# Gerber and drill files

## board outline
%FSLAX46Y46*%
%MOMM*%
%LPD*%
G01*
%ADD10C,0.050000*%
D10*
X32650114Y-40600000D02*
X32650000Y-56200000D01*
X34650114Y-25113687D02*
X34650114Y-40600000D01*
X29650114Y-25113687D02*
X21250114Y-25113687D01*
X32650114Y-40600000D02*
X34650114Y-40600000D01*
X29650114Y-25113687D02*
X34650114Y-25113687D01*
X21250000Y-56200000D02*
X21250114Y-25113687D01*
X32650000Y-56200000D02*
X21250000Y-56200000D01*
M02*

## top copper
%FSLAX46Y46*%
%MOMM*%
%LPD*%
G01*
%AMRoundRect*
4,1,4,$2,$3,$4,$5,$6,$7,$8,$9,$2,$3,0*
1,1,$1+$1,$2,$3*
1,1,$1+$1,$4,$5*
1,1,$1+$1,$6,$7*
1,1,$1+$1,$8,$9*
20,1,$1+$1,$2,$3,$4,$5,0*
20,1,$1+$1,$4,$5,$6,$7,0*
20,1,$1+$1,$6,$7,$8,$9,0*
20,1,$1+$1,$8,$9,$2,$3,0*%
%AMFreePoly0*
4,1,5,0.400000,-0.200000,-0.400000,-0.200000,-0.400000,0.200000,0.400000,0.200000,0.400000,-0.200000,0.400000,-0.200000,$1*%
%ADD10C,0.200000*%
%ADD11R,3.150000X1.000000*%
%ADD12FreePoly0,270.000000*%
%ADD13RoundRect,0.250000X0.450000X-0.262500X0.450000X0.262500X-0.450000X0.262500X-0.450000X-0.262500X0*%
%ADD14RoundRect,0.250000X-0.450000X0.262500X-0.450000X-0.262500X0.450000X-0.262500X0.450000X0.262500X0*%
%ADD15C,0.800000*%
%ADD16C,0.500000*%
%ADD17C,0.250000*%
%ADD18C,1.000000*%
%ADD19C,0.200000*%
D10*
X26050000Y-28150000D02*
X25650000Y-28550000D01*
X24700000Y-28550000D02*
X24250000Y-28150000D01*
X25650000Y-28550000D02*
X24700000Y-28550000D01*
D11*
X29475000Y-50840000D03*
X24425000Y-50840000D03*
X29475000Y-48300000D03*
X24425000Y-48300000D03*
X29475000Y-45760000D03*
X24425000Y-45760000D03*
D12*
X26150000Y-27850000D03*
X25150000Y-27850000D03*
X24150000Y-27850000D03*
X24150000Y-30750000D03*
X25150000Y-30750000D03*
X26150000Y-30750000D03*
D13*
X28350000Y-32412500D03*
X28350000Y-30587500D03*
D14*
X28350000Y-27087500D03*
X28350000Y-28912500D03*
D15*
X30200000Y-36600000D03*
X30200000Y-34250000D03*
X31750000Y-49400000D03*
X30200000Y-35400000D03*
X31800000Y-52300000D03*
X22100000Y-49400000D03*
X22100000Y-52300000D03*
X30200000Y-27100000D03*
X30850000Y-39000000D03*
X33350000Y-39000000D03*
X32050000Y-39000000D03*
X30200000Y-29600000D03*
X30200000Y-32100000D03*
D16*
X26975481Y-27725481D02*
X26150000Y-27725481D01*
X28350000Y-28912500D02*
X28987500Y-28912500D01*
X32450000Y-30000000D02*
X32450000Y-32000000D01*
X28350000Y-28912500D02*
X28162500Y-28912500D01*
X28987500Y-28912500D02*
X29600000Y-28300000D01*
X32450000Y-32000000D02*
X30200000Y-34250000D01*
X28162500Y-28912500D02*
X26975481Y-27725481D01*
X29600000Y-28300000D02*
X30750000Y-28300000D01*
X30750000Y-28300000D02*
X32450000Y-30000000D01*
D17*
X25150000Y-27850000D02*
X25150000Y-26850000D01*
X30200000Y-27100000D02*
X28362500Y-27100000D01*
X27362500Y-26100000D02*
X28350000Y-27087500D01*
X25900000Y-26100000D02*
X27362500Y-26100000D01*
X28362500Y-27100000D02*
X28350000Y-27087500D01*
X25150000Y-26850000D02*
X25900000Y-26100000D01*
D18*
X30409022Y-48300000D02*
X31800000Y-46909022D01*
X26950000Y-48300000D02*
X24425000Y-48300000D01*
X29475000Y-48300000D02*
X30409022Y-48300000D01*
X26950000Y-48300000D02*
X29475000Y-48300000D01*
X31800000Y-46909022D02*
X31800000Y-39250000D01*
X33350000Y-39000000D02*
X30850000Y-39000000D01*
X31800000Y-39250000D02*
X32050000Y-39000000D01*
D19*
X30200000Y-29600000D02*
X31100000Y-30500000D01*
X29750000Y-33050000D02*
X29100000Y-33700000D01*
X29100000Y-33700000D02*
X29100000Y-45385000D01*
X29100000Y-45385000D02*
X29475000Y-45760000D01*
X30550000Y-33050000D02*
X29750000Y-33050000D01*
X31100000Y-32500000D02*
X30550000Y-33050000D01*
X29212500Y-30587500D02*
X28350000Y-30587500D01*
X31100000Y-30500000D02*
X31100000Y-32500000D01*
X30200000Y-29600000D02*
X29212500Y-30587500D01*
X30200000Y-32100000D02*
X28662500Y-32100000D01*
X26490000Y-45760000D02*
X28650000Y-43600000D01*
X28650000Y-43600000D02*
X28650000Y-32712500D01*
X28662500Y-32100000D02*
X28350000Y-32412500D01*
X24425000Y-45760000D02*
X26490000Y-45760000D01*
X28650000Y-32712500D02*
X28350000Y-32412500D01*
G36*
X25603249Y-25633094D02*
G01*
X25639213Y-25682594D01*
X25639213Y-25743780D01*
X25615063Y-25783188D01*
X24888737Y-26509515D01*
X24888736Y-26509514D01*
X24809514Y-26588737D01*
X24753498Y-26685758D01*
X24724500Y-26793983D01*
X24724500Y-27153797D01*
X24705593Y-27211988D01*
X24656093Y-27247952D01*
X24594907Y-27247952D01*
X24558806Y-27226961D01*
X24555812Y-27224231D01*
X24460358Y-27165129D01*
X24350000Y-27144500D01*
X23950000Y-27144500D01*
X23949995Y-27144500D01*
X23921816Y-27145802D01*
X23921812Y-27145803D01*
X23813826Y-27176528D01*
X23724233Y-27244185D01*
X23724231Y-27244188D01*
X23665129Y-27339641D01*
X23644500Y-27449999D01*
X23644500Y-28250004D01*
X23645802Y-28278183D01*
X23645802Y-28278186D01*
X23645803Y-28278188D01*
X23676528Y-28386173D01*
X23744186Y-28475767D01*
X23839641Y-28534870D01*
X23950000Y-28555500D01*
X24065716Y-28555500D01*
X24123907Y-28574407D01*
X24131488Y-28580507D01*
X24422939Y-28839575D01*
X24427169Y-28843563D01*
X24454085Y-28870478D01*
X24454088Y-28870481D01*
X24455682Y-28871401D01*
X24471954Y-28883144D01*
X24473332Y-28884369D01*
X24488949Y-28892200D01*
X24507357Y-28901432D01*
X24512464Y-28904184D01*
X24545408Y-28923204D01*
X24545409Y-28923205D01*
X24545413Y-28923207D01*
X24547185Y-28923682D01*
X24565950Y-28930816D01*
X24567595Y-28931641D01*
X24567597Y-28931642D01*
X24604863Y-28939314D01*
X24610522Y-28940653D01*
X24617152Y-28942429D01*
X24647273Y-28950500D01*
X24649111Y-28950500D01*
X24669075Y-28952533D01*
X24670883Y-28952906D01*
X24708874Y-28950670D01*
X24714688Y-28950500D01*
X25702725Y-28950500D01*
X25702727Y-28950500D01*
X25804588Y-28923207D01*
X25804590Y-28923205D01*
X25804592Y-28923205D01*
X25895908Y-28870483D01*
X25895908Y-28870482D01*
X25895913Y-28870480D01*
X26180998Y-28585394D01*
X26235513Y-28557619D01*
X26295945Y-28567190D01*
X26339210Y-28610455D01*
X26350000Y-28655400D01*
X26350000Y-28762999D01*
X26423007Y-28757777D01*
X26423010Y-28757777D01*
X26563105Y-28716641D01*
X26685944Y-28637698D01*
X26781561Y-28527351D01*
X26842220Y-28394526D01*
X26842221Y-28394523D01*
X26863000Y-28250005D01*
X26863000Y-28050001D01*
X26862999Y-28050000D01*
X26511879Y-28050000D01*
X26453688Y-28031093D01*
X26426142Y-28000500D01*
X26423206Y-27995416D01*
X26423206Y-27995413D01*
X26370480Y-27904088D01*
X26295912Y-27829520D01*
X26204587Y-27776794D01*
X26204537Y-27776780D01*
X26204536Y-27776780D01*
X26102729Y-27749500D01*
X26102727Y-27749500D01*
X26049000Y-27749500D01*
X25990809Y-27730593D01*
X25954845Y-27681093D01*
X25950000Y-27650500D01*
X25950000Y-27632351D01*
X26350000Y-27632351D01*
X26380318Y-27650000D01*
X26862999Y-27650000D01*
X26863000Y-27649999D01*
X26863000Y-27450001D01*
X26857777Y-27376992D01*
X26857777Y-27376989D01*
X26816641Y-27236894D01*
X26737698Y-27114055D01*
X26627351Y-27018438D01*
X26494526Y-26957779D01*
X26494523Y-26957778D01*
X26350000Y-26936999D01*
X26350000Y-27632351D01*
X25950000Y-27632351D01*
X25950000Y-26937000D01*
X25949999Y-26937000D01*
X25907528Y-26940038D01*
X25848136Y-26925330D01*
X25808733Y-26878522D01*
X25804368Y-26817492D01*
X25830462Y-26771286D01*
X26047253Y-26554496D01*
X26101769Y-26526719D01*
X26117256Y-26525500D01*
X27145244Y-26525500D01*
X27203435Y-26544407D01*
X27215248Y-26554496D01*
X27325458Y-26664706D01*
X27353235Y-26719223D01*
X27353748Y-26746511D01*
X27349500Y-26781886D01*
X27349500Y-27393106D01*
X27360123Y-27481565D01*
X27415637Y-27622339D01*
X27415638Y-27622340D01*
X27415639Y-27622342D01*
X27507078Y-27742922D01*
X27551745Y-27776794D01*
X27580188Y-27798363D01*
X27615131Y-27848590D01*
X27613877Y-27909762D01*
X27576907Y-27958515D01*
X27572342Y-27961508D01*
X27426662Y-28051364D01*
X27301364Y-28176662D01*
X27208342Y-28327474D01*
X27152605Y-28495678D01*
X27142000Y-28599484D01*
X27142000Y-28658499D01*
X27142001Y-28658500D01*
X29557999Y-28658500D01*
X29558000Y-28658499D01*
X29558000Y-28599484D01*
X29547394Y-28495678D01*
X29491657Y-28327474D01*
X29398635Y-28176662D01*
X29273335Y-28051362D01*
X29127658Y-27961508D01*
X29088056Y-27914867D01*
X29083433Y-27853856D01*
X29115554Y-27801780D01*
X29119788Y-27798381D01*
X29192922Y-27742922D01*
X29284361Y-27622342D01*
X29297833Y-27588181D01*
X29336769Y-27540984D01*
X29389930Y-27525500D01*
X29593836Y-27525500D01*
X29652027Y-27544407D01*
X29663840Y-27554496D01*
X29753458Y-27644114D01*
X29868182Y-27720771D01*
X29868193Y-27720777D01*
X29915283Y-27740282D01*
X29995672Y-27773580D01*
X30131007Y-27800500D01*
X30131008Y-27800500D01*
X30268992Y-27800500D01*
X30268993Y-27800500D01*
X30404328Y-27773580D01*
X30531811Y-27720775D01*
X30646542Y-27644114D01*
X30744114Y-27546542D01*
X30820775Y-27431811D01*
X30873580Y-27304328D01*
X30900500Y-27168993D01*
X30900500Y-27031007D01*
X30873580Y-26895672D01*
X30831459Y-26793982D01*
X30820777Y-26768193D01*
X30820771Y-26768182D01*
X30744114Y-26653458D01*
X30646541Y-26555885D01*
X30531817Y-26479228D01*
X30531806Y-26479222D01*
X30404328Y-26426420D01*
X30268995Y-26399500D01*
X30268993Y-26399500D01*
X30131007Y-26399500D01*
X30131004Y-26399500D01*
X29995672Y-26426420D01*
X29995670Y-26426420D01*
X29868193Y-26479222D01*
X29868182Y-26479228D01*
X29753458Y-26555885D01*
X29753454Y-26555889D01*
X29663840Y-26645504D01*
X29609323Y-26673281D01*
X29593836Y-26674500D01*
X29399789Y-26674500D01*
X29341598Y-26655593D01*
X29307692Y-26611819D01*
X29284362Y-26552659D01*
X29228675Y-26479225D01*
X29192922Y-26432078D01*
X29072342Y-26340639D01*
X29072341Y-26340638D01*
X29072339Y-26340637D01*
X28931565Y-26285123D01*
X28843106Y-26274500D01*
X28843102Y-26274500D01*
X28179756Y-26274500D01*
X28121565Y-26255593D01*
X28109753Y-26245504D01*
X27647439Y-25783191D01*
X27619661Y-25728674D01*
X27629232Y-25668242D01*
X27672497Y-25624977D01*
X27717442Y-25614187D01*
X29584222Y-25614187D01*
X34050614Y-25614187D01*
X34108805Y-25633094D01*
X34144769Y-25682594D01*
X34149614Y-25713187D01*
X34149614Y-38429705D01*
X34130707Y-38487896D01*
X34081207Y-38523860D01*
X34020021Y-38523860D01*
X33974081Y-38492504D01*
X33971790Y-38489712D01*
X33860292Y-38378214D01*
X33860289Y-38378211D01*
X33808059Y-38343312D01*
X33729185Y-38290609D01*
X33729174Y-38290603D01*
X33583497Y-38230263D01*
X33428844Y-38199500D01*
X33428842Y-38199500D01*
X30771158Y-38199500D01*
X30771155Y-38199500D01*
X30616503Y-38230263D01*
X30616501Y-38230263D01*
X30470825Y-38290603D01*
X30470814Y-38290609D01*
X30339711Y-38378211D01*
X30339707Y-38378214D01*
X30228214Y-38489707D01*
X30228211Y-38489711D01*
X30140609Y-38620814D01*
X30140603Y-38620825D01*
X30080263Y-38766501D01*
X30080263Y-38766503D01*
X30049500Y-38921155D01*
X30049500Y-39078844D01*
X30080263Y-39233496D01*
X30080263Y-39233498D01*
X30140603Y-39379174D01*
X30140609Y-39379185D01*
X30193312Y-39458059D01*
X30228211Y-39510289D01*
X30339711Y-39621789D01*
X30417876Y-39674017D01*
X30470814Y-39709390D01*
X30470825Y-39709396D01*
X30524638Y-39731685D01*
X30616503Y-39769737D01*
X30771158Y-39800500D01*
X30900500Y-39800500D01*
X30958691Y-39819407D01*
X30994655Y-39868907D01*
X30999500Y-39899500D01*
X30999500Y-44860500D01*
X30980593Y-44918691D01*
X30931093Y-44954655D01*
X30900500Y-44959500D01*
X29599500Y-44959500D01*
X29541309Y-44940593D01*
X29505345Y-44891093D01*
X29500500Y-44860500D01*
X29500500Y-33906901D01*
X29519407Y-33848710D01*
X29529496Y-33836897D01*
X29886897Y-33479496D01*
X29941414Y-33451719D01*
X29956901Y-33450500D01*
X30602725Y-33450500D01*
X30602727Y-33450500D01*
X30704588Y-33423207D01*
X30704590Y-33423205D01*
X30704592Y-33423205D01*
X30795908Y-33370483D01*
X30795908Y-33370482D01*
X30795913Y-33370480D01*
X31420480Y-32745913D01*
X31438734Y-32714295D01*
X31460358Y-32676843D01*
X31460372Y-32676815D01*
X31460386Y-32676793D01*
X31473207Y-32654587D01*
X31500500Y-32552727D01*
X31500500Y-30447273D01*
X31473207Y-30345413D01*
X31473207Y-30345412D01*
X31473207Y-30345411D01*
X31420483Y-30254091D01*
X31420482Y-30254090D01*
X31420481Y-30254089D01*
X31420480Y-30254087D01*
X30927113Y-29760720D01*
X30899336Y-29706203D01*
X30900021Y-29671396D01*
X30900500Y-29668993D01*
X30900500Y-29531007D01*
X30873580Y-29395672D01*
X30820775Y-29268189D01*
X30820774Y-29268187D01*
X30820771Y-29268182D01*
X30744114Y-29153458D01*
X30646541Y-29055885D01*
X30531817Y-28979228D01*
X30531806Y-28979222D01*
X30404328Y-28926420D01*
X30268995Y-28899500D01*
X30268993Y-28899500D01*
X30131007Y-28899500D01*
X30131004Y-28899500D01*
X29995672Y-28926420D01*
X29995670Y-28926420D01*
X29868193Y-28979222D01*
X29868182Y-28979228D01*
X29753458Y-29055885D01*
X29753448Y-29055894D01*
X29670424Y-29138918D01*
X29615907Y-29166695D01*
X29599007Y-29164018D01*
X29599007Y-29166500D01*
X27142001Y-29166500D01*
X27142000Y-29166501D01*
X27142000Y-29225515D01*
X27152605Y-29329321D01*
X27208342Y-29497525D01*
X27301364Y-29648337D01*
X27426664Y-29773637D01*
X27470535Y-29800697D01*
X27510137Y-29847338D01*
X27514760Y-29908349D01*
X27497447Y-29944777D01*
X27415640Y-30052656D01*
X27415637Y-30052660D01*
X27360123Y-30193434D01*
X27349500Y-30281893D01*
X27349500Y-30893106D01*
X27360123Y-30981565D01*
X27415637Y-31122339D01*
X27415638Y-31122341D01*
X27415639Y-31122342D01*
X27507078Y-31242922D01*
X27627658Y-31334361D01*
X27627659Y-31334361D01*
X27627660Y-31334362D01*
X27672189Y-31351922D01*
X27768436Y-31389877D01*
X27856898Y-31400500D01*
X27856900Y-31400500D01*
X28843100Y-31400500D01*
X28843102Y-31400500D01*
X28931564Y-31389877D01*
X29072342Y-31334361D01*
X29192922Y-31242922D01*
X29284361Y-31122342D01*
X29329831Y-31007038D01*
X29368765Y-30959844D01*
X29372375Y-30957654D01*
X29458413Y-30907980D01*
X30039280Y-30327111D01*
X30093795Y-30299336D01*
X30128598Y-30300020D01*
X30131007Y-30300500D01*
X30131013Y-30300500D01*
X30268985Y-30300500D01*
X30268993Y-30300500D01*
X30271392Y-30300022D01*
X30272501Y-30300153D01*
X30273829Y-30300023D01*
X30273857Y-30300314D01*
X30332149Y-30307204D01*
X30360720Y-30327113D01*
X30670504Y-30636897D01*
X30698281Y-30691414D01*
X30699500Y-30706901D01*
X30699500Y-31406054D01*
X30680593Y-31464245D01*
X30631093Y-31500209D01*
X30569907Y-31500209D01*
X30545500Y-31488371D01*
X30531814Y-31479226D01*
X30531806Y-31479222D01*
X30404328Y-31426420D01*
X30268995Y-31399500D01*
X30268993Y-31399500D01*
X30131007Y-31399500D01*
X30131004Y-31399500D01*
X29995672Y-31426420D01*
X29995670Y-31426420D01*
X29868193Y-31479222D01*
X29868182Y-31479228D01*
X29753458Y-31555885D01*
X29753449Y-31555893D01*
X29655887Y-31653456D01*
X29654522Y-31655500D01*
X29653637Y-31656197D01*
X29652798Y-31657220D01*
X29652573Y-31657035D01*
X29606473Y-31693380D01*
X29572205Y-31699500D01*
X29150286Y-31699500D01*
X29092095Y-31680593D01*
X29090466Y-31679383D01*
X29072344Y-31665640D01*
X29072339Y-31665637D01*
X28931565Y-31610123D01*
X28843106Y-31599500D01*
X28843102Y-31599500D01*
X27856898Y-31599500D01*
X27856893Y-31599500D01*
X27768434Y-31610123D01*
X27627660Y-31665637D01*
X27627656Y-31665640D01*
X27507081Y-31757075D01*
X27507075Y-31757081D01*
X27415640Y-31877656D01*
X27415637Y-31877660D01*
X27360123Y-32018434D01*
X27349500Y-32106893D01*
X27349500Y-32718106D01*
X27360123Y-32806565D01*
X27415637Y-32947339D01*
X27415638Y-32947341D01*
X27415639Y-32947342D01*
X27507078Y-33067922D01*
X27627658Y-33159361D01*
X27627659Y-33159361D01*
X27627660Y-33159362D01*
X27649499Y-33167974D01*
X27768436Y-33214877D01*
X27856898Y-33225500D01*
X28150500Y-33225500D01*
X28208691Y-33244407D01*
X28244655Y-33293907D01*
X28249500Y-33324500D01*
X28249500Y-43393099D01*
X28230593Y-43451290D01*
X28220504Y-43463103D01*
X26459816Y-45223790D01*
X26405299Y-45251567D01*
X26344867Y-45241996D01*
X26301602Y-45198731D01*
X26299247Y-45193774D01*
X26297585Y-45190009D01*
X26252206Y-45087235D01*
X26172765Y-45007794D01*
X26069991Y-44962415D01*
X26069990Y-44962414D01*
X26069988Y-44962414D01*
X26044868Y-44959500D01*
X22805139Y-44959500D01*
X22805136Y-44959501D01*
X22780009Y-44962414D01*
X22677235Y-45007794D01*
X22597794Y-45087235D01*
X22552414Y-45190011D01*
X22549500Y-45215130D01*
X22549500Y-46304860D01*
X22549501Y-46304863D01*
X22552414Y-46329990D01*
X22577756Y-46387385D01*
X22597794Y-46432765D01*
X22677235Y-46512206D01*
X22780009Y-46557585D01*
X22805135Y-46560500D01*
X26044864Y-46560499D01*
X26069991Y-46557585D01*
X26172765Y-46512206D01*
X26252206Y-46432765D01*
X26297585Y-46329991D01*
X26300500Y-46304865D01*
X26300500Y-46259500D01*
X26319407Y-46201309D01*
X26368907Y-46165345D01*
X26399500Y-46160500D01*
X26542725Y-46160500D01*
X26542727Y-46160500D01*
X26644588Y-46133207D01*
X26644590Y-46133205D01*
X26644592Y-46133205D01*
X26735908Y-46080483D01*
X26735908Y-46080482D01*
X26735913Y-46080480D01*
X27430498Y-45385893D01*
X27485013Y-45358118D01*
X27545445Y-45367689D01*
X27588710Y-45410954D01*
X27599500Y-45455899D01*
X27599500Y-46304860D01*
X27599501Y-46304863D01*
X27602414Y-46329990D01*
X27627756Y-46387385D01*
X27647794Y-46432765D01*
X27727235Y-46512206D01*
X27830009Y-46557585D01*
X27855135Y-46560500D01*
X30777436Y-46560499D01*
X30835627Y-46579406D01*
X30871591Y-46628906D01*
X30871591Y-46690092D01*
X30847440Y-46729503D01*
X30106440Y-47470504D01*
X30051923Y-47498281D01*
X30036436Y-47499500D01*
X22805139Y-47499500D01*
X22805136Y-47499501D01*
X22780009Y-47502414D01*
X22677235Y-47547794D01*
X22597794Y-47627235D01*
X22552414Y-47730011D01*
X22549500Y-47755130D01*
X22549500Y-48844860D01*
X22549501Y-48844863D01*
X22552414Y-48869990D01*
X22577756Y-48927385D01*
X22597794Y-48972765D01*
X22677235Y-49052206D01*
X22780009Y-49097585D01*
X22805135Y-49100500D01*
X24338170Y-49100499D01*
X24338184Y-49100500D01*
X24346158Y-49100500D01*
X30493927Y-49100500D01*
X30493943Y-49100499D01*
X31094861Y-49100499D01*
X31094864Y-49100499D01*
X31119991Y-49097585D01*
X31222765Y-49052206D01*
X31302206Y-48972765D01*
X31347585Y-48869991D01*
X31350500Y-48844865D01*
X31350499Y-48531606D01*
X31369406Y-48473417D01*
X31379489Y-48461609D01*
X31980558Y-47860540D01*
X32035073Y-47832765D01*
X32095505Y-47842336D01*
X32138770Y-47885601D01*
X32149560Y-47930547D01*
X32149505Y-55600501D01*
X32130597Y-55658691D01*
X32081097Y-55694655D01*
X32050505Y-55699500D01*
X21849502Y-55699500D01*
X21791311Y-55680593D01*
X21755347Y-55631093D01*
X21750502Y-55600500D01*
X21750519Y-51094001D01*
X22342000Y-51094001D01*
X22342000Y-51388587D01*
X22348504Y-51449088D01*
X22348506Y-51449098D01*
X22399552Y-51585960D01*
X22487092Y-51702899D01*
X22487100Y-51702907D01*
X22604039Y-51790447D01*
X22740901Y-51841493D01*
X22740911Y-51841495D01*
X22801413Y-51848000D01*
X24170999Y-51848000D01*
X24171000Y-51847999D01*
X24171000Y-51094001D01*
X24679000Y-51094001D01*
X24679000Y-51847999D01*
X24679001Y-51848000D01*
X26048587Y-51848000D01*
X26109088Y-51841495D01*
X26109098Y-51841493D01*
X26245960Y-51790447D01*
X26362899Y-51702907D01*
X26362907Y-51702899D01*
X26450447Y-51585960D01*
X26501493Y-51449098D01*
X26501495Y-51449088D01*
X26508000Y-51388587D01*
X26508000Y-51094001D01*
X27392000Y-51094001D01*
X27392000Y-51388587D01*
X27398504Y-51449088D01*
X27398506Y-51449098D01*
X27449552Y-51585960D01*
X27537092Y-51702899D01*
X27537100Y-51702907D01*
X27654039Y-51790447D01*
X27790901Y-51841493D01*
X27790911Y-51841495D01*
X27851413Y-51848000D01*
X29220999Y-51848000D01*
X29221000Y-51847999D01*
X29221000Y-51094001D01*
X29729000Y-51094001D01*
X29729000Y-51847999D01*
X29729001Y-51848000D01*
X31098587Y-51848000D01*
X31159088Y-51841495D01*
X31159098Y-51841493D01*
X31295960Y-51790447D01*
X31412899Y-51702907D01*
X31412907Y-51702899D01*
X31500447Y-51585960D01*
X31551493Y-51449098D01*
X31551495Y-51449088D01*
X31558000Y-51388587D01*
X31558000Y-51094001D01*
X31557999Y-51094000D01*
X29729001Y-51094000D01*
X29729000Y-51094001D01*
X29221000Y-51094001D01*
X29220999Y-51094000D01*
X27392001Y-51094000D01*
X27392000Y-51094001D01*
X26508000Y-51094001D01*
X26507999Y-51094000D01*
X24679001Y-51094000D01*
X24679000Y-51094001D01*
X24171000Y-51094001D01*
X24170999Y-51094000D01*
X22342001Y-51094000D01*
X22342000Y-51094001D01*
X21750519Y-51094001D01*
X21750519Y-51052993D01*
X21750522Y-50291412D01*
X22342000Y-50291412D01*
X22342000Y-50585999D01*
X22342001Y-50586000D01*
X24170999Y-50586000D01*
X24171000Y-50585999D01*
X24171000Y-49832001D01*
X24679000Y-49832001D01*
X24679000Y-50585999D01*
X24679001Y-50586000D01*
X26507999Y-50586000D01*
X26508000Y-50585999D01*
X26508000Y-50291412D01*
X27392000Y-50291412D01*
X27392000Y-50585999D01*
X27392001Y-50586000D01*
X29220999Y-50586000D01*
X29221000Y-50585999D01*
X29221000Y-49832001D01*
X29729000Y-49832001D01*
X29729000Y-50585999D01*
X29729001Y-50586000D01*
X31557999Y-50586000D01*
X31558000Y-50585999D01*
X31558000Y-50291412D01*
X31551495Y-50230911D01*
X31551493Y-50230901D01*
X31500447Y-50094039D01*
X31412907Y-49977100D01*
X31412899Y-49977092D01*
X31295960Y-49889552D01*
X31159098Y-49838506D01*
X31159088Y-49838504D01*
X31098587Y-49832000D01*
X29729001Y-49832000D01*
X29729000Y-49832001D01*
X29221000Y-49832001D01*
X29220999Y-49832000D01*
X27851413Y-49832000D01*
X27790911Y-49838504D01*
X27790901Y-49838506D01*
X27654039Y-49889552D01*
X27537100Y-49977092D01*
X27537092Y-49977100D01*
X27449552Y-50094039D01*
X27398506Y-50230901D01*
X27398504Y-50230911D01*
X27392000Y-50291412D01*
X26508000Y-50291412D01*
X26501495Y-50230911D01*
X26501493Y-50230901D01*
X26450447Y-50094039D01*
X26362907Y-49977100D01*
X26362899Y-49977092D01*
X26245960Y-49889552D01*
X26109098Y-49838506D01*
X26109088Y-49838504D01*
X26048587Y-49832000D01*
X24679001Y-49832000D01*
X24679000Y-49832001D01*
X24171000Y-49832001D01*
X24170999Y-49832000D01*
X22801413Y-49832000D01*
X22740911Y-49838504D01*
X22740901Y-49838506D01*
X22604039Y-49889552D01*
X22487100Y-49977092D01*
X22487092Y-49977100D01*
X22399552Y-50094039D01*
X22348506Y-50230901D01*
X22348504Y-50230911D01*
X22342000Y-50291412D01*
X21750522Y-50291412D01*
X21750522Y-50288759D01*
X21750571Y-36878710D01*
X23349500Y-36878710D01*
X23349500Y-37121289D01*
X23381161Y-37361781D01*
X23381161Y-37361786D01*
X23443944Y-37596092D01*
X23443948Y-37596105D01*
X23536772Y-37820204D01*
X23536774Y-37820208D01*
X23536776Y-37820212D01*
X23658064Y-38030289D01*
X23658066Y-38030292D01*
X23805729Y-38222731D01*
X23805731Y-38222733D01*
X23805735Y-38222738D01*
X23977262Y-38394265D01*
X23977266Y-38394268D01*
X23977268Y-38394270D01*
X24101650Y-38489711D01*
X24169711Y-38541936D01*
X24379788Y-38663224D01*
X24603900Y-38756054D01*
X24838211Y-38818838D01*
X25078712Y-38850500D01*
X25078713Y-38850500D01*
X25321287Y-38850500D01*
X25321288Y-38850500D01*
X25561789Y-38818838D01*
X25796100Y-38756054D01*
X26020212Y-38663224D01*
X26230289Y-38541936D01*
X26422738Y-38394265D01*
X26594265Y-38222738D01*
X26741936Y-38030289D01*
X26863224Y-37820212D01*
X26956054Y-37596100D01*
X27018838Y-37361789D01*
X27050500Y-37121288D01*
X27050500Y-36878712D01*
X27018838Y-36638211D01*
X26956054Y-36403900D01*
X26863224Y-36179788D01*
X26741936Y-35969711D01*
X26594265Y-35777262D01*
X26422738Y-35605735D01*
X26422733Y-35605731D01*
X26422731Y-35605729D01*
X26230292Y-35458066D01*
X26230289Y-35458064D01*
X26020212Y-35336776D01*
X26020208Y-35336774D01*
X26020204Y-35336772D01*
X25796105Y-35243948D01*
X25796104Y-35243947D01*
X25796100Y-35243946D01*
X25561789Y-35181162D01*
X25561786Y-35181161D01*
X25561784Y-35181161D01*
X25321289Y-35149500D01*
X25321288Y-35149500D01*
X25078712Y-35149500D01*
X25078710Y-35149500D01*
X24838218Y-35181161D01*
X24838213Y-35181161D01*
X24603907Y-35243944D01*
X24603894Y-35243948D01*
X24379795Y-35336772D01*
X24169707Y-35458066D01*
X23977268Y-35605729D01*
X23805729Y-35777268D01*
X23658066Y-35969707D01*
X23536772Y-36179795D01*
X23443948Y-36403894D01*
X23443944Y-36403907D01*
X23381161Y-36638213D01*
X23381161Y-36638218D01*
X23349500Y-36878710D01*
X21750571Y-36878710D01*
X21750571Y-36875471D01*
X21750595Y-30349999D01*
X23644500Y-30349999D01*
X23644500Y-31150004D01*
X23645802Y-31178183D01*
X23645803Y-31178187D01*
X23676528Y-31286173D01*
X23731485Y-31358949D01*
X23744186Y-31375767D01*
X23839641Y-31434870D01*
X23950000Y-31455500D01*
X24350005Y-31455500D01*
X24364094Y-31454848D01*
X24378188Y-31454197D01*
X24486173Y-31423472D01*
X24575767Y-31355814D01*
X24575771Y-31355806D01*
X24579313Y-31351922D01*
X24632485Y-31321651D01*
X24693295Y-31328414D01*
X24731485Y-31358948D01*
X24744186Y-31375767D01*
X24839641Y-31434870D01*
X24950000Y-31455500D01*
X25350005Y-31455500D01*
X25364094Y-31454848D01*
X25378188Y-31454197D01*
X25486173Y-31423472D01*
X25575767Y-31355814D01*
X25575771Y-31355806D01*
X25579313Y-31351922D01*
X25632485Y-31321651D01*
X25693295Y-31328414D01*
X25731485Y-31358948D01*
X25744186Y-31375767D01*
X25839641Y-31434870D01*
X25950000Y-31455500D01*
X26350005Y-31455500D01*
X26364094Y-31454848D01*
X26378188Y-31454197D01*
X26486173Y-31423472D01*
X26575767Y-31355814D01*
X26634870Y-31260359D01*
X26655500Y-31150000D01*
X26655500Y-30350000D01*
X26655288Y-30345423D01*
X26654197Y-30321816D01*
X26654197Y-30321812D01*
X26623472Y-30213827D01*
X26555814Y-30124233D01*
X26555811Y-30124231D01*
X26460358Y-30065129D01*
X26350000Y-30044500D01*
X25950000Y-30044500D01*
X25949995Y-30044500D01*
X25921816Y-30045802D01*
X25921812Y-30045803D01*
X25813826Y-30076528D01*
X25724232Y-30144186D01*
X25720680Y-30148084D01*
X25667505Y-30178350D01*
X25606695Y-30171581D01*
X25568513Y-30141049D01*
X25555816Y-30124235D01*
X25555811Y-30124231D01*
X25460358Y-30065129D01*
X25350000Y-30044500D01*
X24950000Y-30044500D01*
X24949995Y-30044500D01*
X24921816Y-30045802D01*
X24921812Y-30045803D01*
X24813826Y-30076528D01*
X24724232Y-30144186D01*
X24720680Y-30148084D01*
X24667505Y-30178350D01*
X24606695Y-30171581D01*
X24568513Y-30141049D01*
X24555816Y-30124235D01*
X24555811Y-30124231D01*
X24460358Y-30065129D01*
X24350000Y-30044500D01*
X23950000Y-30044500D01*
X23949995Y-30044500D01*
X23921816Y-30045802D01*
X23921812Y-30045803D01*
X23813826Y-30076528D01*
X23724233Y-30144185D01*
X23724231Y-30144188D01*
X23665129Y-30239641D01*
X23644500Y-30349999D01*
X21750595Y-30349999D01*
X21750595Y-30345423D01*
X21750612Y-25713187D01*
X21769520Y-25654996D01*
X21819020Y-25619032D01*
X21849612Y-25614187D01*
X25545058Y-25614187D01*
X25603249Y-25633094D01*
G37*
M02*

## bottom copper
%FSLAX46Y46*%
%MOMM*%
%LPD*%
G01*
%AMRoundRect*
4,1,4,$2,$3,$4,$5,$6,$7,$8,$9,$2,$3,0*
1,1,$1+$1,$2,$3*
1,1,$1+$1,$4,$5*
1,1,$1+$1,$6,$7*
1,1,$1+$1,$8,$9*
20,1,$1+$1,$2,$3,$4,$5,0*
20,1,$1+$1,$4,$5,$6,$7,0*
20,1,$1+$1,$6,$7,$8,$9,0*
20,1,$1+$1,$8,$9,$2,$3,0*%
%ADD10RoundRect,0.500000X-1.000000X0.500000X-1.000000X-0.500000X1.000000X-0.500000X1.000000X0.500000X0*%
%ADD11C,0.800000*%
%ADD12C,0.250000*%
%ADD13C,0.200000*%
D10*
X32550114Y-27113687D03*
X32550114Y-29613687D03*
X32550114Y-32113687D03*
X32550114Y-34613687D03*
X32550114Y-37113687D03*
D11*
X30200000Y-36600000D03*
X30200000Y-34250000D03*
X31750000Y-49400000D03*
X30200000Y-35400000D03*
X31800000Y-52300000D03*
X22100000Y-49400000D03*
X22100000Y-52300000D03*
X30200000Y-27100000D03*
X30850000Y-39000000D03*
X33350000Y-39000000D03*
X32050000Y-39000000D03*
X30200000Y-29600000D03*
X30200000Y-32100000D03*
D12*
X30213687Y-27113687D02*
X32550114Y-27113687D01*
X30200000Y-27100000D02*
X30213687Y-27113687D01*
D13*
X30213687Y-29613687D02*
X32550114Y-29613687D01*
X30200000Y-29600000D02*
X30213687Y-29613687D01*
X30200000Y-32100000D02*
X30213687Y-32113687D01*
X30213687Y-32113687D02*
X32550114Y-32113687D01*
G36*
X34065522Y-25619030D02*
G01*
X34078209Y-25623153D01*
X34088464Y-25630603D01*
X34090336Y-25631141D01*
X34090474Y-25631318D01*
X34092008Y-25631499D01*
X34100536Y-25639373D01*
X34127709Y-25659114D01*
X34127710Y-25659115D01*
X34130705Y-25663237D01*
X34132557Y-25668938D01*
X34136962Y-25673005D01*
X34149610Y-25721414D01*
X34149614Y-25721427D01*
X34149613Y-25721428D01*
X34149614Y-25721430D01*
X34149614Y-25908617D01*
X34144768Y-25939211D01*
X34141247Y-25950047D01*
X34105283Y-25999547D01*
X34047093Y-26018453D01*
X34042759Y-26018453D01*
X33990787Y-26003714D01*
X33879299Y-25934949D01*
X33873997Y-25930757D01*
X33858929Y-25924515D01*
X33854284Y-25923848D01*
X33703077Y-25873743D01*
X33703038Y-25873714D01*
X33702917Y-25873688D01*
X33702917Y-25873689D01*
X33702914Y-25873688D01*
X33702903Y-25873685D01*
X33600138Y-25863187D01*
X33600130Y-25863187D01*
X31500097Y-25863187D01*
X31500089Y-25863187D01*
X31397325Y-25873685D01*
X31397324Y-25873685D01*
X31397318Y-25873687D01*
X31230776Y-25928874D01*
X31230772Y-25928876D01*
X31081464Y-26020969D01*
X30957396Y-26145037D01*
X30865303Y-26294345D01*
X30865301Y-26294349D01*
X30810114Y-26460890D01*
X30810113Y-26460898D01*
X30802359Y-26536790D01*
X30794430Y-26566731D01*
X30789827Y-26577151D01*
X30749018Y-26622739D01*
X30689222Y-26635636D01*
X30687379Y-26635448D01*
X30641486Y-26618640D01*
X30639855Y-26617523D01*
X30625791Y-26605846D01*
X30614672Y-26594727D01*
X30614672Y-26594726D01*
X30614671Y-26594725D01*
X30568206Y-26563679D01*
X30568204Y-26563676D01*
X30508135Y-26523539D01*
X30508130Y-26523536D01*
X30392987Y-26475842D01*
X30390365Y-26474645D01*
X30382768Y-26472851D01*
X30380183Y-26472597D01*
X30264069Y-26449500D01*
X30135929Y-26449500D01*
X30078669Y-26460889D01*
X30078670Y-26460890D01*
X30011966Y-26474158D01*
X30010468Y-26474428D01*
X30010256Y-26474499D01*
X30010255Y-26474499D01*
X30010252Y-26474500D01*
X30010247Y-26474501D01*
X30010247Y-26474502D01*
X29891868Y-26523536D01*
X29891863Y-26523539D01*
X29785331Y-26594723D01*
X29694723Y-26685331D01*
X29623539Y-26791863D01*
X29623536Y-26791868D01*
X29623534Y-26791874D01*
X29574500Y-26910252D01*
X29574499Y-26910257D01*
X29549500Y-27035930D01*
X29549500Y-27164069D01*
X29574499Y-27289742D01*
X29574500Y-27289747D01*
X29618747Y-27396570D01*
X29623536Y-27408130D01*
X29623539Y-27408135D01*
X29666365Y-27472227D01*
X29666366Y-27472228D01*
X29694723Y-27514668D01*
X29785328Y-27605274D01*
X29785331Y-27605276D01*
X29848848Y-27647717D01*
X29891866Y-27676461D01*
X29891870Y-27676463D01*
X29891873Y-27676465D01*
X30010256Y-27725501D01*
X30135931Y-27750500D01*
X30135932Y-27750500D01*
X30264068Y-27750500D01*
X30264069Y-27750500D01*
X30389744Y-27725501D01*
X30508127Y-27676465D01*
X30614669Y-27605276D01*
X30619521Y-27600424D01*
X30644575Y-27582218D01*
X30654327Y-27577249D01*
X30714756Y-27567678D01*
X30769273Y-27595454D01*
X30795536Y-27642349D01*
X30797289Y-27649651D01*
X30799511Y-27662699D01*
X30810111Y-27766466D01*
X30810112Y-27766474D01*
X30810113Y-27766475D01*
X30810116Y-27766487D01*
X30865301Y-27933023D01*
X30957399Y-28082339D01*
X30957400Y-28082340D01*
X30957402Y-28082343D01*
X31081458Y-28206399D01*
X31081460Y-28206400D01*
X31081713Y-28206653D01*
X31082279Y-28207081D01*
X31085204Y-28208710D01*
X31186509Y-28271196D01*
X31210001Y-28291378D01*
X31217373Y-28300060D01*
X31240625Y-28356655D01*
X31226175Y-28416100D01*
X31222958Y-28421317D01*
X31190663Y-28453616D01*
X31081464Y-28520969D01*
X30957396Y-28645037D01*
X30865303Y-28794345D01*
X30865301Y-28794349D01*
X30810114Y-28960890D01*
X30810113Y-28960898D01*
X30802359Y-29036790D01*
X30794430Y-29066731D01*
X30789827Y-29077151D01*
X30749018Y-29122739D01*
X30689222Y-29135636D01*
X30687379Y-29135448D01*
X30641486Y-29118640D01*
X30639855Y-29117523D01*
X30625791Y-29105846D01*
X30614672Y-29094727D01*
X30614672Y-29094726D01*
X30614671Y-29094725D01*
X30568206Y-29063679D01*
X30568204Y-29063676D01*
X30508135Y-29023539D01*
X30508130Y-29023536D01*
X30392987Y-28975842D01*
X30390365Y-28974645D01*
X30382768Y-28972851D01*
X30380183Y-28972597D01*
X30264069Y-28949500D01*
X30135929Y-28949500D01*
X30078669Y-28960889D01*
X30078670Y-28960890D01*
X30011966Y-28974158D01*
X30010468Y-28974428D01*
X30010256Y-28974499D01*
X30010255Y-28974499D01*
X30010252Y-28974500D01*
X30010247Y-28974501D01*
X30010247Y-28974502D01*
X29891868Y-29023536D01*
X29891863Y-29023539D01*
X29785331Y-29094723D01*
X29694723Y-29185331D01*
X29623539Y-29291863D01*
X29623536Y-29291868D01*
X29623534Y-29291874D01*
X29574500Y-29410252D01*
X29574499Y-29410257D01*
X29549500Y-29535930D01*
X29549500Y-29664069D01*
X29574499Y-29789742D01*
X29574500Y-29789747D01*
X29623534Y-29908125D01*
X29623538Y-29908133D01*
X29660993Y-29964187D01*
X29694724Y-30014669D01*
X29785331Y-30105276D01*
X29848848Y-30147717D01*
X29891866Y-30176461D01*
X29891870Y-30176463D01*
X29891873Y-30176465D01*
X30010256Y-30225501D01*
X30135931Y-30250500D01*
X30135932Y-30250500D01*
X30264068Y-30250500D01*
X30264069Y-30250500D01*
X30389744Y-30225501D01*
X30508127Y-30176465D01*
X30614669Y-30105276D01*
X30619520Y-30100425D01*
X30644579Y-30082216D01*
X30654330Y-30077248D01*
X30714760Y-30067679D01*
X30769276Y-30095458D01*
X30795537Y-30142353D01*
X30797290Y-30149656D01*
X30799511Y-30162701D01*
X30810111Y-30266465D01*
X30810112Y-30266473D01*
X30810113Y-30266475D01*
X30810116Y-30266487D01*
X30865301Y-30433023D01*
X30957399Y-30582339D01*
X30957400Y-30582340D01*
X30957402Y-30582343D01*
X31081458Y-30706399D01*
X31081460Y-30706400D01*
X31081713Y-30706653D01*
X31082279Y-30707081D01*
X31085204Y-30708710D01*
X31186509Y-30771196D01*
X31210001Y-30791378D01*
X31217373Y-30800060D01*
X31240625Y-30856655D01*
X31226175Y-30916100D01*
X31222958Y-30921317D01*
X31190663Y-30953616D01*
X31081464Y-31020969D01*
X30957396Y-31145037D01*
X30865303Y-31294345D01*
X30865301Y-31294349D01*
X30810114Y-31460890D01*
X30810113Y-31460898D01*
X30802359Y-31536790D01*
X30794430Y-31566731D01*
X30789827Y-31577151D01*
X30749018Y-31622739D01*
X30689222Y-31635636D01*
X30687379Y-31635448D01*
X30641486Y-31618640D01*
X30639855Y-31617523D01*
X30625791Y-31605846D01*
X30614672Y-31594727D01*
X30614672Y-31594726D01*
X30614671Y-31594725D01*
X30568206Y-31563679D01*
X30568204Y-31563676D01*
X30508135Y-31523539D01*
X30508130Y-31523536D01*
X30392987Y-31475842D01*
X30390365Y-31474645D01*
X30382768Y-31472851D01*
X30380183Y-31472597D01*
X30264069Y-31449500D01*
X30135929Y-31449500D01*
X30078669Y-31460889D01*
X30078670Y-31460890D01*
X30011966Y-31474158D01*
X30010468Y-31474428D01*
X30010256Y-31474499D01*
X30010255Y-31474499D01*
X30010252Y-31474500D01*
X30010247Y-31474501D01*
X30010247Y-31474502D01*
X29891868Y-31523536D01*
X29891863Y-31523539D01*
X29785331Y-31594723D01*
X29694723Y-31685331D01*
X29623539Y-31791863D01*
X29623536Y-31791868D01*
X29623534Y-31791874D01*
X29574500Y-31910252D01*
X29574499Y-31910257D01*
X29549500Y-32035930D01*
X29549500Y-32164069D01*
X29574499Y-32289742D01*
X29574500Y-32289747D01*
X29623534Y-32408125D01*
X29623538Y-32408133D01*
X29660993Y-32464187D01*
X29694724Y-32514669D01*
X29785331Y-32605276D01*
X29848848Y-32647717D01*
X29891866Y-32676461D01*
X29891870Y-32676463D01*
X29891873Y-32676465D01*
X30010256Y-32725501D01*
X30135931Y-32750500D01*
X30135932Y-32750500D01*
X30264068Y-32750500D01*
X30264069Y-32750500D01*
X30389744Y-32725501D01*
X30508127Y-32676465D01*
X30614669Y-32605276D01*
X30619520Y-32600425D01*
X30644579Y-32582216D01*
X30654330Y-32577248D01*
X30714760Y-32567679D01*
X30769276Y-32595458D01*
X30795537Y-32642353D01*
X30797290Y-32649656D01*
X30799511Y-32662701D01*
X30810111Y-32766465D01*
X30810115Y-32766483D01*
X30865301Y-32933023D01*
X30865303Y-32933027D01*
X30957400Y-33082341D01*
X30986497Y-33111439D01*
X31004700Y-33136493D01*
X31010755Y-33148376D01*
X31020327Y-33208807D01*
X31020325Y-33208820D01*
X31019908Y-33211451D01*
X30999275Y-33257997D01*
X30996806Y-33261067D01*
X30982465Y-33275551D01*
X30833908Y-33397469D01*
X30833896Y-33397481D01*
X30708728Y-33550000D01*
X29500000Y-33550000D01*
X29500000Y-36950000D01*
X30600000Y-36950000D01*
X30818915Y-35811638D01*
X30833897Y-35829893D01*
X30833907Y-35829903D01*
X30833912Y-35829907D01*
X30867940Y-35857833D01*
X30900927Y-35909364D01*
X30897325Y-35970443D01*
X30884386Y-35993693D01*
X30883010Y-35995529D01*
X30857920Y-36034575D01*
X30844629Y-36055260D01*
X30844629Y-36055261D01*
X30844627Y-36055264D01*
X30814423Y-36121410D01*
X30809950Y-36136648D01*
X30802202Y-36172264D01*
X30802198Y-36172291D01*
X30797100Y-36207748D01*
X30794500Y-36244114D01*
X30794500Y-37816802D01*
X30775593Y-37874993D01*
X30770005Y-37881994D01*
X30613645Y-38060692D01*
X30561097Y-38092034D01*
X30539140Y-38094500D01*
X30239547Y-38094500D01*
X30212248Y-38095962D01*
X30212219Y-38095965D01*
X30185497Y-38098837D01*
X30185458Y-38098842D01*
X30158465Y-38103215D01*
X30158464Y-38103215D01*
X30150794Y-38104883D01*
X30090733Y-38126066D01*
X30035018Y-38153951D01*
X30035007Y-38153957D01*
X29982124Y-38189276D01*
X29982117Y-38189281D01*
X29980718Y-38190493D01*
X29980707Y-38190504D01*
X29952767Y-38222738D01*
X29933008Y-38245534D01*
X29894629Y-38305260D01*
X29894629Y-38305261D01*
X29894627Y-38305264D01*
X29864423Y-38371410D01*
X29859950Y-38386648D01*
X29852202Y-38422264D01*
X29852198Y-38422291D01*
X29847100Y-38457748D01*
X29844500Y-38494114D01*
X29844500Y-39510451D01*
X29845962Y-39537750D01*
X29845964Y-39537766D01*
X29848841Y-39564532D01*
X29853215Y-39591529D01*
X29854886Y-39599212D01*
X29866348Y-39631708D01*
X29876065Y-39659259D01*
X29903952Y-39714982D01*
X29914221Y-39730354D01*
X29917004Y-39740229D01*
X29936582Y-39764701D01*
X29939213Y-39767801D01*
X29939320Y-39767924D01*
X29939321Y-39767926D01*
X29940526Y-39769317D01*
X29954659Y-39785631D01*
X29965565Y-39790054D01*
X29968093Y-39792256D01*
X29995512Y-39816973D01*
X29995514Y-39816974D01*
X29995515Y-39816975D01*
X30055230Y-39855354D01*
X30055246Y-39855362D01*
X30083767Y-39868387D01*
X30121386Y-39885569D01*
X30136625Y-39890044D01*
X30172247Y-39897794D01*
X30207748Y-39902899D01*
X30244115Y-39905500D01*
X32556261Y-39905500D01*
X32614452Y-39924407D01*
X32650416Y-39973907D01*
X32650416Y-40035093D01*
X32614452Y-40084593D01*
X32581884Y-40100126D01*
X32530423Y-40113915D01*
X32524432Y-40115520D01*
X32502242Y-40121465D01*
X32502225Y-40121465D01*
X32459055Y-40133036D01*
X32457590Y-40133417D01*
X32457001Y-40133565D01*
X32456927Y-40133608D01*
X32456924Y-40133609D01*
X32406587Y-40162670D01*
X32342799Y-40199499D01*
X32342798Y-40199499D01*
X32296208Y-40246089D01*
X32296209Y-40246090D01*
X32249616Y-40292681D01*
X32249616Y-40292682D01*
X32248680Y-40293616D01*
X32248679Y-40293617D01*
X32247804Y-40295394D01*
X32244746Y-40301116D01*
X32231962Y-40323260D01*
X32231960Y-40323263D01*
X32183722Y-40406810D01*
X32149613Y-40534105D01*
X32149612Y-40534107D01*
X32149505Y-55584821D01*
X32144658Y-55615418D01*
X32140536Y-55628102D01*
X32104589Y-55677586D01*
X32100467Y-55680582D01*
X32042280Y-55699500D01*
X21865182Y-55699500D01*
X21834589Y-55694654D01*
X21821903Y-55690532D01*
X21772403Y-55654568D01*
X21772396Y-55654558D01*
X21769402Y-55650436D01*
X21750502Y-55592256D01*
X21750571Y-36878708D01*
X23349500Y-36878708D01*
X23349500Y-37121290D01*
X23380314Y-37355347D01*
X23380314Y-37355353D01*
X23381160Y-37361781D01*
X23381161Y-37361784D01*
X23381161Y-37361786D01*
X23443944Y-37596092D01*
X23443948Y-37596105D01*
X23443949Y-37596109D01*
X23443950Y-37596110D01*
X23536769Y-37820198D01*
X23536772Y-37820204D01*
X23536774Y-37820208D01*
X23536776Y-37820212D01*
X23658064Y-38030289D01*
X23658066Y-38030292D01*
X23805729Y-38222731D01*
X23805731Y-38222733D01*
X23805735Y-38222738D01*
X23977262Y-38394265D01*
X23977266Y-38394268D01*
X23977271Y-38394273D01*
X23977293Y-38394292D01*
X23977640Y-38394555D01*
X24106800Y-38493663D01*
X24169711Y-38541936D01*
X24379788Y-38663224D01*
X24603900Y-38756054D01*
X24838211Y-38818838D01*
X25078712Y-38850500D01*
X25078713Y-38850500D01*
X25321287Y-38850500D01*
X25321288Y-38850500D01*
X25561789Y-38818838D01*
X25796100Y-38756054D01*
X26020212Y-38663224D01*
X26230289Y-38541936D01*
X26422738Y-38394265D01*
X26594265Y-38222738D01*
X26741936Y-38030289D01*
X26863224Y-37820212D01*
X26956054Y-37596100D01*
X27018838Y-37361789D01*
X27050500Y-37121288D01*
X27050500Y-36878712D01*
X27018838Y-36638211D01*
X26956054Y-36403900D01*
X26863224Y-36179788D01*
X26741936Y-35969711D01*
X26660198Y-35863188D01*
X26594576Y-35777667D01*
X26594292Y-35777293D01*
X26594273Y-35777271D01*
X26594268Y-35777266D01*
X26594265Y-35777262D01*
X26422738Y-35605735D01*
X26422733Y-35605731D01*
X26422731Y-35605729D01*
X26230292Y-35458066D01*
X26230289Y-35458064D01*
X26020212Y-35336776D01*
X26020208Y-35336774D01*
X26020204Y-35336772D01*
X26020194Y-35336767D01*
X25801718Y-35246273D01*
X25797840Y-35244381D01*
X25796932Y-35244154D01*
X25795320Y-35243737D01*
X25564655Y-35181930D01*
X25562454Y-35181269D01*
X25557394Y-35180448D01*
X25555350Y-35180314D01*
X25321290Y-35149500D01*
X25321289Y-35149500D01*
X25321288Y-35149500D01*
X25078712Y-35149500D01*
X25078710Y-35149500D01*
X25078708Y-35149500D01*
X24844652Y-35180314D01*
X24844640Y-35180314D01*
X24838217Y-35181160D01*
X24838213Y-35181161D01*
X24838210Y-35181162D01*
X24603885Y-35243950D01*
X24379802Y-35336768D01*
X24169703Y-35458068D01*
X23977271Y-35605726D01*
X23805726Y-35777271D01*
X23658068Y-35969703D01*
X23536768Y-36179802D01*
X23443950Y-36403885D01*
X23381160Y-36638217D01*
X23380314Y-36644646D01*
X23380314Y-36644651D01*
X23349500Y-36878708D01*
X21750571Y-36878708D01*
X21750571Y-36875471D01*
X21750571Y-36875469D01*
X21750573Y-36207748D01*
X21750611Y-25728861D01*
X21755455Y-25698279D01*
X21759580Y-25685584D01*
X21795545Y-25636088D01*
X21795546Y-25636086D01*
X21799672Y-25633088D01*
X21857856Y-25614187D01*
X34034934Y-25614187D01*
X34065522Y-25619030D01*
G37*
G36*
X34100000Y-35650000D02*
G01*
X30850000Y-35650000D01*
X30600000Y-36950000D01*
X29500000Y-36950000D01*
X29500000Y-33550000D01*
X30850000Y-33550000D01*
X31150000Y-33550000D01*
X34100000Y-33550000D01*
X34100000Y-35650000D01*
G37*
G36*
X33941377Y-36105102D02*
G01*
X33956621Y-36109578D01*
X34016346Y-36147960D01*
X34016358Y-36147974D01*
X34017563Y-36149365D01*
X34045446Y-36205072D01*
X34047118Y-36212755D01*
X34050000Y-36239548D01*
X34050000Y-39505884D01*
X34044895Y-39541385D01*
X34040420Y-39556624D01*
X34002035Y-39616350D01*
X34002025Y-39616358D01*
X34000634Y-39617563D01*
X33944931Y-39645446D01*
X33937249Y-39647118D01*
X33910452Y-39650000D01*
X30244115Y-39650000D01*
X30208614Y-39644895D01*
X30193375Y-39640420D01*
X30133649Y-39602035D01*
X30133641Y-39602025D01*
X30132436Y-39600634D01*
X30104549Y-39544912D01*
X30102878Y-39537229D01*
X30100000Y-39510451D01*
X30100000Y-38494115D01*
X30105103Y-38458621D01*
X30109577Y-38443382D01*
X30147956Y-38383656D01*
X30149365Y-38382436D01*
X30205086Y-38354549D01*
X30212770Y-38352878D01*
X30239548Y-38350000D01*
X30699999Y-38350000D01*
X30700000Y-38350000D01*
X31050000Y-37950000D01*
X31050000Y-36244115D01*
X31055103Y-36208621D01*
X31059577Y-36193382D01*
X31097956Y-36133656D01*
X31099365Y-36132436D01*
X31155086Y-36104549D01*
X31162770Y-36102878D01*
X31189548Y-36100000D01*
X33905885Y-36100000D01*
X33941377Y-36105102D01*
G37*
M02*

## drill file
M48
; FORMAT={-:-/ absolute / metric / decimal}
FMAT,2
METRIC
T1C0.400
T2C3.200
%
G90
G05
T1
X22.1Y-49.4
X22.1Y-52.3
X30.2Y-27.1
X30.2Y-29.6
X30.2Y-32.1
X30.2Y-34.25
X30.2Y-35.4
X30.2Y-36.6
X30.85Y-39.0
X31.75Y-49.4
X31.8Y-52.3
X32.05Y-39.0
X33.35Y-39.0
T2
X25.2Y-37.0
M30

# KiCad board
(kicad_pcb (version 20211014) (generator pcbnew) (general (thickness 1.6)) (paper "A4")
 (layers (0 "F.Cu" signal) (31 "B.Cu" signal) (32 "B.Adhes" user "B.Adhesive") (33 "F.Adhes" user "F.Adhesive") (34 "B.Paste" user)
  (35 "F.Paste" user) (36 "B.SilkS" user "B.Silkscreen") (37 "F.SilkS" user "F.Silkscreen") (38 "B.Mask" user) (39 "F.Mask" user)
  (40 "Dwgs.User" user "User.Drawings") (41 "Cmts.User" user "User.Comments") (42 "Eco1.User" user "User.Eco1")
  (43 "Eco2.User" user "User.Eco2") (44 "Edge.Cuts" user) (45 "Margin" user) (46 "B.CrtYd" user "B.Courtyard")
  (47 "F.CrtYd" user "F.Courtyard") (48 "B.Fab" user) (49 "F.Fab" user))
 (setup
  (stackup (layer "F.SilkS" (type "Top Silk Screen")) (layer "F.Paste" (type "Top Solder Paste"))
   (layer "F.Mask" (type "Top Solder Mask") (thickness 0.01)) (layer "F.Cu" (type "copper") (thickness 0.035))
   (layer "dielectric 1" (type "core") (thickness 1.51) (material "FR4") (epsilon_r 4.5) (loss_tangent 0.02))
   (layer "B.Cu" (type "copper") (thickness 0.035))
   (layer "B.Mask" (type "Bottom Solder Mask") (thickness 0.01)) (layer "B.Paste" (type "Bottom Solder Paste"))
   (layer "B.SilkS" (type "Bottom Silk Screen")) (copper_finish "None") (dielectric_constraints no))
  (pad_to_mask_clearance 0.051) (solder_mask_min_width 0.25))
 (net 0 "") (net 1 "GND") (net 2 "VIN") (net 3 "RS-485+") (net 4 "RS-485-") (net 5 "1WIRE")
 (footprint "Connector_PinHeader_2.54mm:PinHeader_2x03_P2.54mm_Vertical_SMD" (layer "F.Cu") (at 26.95 48.3 180)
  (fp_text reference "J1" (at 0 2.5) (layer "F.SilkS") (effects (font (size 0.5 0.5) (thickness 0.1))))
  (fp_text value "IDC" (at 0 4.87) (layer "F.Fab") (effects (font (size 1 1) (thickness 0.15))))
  (pad "1" smd rect (at -2.525 -2.54 180) (size 3.15 1) (layers "F.Cu" "F.Paste" "F.Mask") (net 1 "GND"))
  (pad "2" smd rect (at 2.525 -2.54 180) (size 3.15 1) (layers "F.Cu" "F.Paste" "F.Mask") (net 1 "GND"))
  (pad "3" smd rect (at -2.525 0 180) (size 3.15 1) (layers "F.Cu" "F.Paste" "F.Mask") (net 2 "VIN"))
  (pad "4" smd rect (at 2.525 0 180) (size 3.15 1) (layers "F.Cu" "F.Paste" "F.Mask") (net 2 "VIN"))
  (pad "5" smd rect (at -2.525 2.54 180) (size 3.15 1) (layers "F.Cu" "F.Paste" "F.Mask") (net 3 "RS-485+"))
  (pad "6" smd rect (at 2.525 2.54 180) (size 3.15 1) (layers "F.Cu" "F.Paste" "F.Mask") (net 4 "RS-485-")))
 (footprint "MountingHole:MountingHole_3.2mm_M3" (layer "F.Cu") (at 25.2 37)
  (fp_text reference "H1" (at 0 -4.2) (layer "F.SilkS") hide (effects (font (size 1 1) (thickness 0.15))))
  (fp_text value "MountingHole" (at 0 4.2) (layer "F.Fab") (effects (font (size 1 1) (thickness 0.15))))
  (pad "" np_thru_hole circle (at 0 0) (size 3.2 3.2) (drill 3.2) (layers *.Cu *.Mask)))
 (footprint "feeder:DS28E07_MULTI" (layer "F.Cu") (at 25.15 29.3 -90)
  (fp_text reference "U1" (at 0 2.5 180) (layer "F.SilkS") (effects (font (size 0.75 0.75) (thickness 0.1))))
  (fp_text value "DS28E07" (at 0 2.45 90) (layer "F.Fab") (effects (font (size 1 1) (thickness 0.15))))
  (fp_line (start -1.15 -0.9) (end -0.75 -0.5) (layer "F.Cu") (width 0.2))
  (fp_line (start -0.75 0.45) (end -1.15 0.9) (layer "F.Cu") (width 0.2))
  (fp_line (start -0.75 -0.5) (end -0.75 0.45) (layer "F.Cu") (width 0.2))
  (pad "1" smd custom (at -1.45 -1 270) (size 0.8 0.4) (layers "F.Cu" "F.Paste" "F.Mask") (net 1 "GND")
   (options (clearance outline) (anchor rect)) (primitives))
  (pad "2" smd custom (at -1.45 0 270) (size 0.8 0.4) (layers "F.Cu" "F.Paste" "F.Mask") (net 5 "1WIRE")
   (options (clearance outline) (anchor rect)) (primitives))
  (pad "3" smd custom (at -1.45 1 270) (size 0.8 0.4) (layers "F.Cu" "F.Paste" "F.Mask") (options (clearance outline) (anchor rect))
   (primitives))
  (pad "4" smd custom (at 1.45 1 270) (size 0.8 0.4) (layers "F.Cu" "F.Paste" "F.Mask") (options (clearance outline) (anchor rect))
   (primitives))
  (pad "5" smd custom (at 1.45 0 270) (size 0.8 0.4) (layers "F.Cu" "F.Paste" "F.Mask") (options (clearance outline) (anchor rect))
   (primitives))
  (pad "6" smd custom (at 1.45 -1 270) (size 0.8 0.4) (layers "F.Cu" "F.Paste" "F.Mask") (options (clearance outline) (anchor rect))
   (primitives)))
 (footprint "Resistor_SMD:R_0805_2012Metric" (layer "F.Cu") (at 28.35 31.5 90)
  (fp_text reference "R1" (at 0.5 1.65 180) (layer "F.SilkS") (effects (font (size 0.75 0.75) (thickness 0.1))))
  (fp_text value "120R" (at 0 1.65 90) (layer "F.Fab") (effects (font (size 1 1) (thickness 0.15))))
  (pad "1" smd roundrect (at -0.9125 0 90) (size 1.025 1.4) (layers "F.Cu" "F.Paste" "F.Mask") (roundrect_rratio 0.243902439)
   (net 4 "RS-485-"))
  (pad "2" smd roundrect (at 0.9125 0 90) (size 1.025 1.4) (layers "F.Cu" "F.Paste" "F.Mask") (roundrect_rratio 0.243902439)
   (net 3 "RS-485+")))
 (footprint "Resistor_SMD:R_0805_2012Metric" (layer "F.Cu") (at 28.35 28 -90)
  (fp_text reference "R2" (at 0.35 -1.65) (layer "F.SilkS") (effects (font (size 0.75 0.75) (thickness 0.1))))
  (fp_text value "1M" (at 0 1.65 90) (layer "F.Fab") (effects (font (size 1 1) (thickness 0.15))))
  (pad "1" smd roundrect (at -0.9125 0 270) (size 1.025 1.4) (layers "F.Cu" "F.Paste" "F.Mask") (roundrect_rratio 0.243902439)
   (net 5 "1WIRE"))
  (pad "2" smd roundrect (at 0.9125 0 270) (size 1.025 1.4) (layers "F.Cu" "F.Paste" "F.Mask") (roundrect_rratio 0.243902439) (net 1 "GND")))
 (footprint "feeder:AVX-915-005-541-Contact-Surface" (layer "B.Cu") (at 32.550114 27.113687 -90)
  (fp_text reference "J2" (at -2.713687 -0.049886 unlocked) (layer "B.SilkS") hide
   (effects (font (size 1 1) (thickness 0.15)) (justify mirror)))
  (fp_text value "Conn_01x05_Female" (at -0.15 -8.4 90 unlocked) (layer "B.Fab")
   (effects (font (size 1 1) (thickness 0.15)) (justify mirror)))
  (pad "1" smd roundrect (at 0 0 270) (size 2 3) (layers "B.Cu" "B.Paste" "B.Mask") (roundrect_rratio 0.25) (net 5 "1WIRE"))
  (pad "2" smd roundrect (at 2.5 0 270) (size 2 3) (layers "B.Cu" "B.Paste" "B.Mask") (roundrect_rratio 0.25) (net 3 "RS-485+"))
  (pad "3" smd roundrect (at 5 0 270) (size 2 3) (layers "B.Cu" "B.Paste" "B.Mask") (roundrect_rratio 0.25) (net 4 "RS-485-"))
  (pad "4" smd roundrect (at 7.5 0 270) (size 2 3) (layers "B.Cu" "B.Paste" "B.Mask") (roundrect_rratio 0.25) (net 1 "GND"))
  (pad "5" smd roundrect (at 10 0 270) (size 2 3) (layers "B.Cu" "B.Paste" "B.Mask") (roundrect_rratio 0.25) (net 2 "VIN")))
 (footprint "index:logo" (layer "B.Cu") (at 26.95 50.5 180)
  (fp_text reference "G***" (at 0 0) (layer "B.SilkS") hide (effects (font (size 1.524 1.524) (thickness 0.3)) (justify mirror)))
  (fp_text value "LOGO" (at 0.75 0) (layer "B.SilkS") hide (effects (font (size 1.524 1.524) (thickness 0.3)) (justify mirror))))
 (gr_line (start 32.650114 40.6) (end 32.65 56.2) (layer "Edge.Cuts") (width 0.05))
 (gr_line (start 34.650114 25.113687) (end 34.650114 40.6) (layer "Edge.Cuts") (width 0.05))
 (gr_line (start 29.650114 25.113687) (end 21.250114 25.113687) (layer "Edge.Cuts") (width 0.05))
 (gr_line (start 32.650114 40.6) (end 34.650114 40.6) (layer "Edge.Cuts") (width 0.05))
 (gr_line (start 29.650114 25.113687) (end 34.650114 25.113687) (layer "Edge.Cuts") (width 0.05))
 (gr_line (start 21.25 56.2) (end 21.250114 25.113687) (layer "Edge.Cuts") (width 0.05))
 (gr_line (start 32.65 56.2) (end 21.25 56.2) (layer "Edge.Cuts") (width 0.05))
 (segment (start 26.975481 27.725481) (end 26.15 27.725481) (width 0.5) (layer "F.Cu") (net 1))
 (segment (start 28.35 28.9125) (end 28.9875 28.9125) (width 0.5) (layer "F.Cu") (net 1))
 (segment (start 32.45 30) (end 32.45 32) (width 0.5) (layer "F.Cu") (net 1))
 (segment (start 28.35 28.9125) (end 28.1625 28.9125) (width 0.5) (layer "F.Cu") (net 1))
 (segment (start 28.9875 28.9125) (end 29.6 28.3) (width 0.5) (layer "F.Cu") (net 1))
 (segment (start 32.45 32) (end 30.2 34.25) (width 0.5) (layer "F.Cu") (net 1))
 (segment (start 28.1625 28.9125) (end 26.975481 27.725481) (width 0.5) (layer "F.Cu") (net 1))
 (segment (start 29.6 28.3) (end 30.75 28.3) (width 0.5) (layer "F.Cu") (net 1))
 (segment (start 30.75 28.3) (end 32.45 30) (width 0.5) (layer "F.Cu") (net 1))
 (via (at 30.2 36.6) (size 0.8) (drill 0.4) (layers "F.Cu" "B.Cu") (free) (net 1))
 (via (at 30.2 34.25) (size 0.8) (drill 0.4) (layers "F.Cu" "B.Cu") (free) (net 1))
 (via (at 31.75 49.4) (size 0.8) (drill 0.4) (layers "F.Cu" "B.Cu") (free) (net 1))
 (via (at 30.2 35.4) (size 0.8) (drill 0.4) (layers "F.Cu" "B.Cu") (free) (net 1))
 (via (at 31.8 52.3) (size 0.8) (drill 0.4) (layers "F.Cu" "B.Cu") (free) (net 1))
 (via (at 22.1 49.4) (size 0.8) (drill 0.4) (layers "F.Cu" "B.Cu") (free) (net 1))
 (via (at 22.1 52.3) (size 0.8) (drill 0.4) (layers "F.Cu" "B.Cu") (free) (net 1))
 (segment (start 25.15 27.85) (end 25.15 26.85) (width 0.25) (layer "F.Cu") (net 5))
 (segment (start 30.2 27.1) (end 28.3625 27.1) (width 0.25) (layer "F.Cu") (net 5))
 (segment (start 27.3625 26.1) (end 28.35 27.0875) (width 0.25) (layer "F.Cu") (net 5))
 (segment (start 25.9 26.1) (end 27.3625 26.1) (width 0.25) (layer "F.Cu") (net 5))
 (segment (start 28.3625 27.1) (end 28.35 27.0875) (width 0.25) (layer "F.Cu") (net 5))
 (segment (start 25.15 26.85) (end 25.9 26.1) (width 0.25) (layer "F.Cu") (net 5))
 (via (at 30.2 27.1) (size 0.8) (drill 0.4) (layers "F.Cu" "B.Cu") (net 5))
 (segment (start 30.213687 27.113687) (end 32.550114 27.113687) (width 0.25) (layer "B.Cu") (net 5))
 (segment (start 30.2 27.1) (end 30.213687 27.113687) (width 0.25) (layer "B.Cu") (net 5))
 (segment (start 30.409022 48.3) (end 31.8 46.909022) (width 1) (layer "F.Cu") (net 2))
 (segment (start 26.95 48.3) (end 24.425 48.3) (width 1) (layer "F.Cu") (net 2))
 (segment (start 29.475 48.3) (end 30.409022 48.3) (width 1) (layer "F.Cu") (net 2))
 (segment (start 26.95 48.3) (end 29.475 48.3) (width 1) (layer "F.Cu") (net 2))
 (segment (start 31.8 46.909022) (end 31.8 39.25) (width 1) (layer "F.Cu") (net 2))
 (segment (start 33.35 39) (end 30.85 39) (width 1) (layer "F.Cu") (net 2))
 (segment (start 31.8 39.25) (end 32.05 39) (width 1) (layer "F.Cu") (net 2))
 (via (at 30.85 39) (size 0.8) (drill 0.4) (layers "F.Cu" "B.Cu") (free) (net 2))
 (via (at 33.35 39) (size 0.8) (drill 0.4) (layers "F.Cu" "B.Cu") (free) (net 2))
 (via (at 32.05 39) (size 0.8) (drill 0.4) (layers "F.Cu" "B.Cu") (free) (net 2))
 (segment (start 30.2 29.6) (end 31.1 30.5) (width 0.2) (layer "F.Cu") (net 3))
 (segment (start 29.75 33.05) (end 29.1 33.7) (width 0.2) (layer "F.Cu") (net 3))
 (segment (start 29.1 33.7) (end 29.1 45.385) (width 0.2) (layer "F.Cu") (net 3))
 (segment (start 29.1 45.385) (end 29.475 45.76) (width 0.2) (layer "F.Cu") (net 3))
 (segment (start 30.55 33.05) (end 29.75 33.05) (width 0.2) (layer "F.Cu") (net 3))
 (segment (start 31.1 32.5) (end 30.55 33.05) (width 0.2) (layer "F.Cu") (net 3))
 (segment (start 29.2125 30.5875) (end 28.35 30.5875) (width 0.2) (layer "F.Cu") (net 3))
 (segment (start 31.1 30.5) (end 31.1 32.5) (width 0.2) (layer "F.Cu") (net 3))
 (segment (start 30.2 29.6) (end 29.2125 30.5875) (width 0.2) (layer "F.Cu") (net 3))
 (via (at 30.2 29.6) (size 0.8) (drill 0.4) (layers "F.Cu" "B.Cu") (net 3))
 (segment (start 30.213687 29.613687) (end 32.550114 29.613687) (width 0.2) (layer "B.Cu") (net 3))
 (segment (start 30.2 29.6) (end 30.213687 29.613687) (width 0.2) (layer "B.Cu") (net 3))
 (segment (start 30.2 32.1) (end 28.6625 32.1) (width 0.2) (layer "F.Cu") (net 4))
 (segment (start 26.49 45.76) (end 28.65 43.6) (width 0.2) (layer "F.Cu") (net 4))
 (segment (start 28.65 43.6) (end 28.65 32.7125) (width 0.2) (layer "F.Cu") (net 4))
 (segment (start 28.6625 32.1) (end 28.35 32.4125) (width 0.2) (layer "F.Cu") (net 4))
 (segment (start 24.425 45.76) (end 26.49 45.76) (width 0.2) (layer "F.Cu") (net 4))
 (segment (start 28.65 32.7125) (end 28.35 32.4125) (width 0.2) (layer "F.Cu") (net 4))
 (via (at 30.2 32.1) (size 0.8) (drill 0.4) (layers "F.Cu" "B.Cu") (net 4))
 (segment (start 30.2 32.1) (end 30.213687 32.113687) (width 0.2) (layer "B.Cu") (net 4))
 (segment (start 30.213687 32.113687) (end 32.550114 32.113687) (width 0.2) (layer "B.Cu") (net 4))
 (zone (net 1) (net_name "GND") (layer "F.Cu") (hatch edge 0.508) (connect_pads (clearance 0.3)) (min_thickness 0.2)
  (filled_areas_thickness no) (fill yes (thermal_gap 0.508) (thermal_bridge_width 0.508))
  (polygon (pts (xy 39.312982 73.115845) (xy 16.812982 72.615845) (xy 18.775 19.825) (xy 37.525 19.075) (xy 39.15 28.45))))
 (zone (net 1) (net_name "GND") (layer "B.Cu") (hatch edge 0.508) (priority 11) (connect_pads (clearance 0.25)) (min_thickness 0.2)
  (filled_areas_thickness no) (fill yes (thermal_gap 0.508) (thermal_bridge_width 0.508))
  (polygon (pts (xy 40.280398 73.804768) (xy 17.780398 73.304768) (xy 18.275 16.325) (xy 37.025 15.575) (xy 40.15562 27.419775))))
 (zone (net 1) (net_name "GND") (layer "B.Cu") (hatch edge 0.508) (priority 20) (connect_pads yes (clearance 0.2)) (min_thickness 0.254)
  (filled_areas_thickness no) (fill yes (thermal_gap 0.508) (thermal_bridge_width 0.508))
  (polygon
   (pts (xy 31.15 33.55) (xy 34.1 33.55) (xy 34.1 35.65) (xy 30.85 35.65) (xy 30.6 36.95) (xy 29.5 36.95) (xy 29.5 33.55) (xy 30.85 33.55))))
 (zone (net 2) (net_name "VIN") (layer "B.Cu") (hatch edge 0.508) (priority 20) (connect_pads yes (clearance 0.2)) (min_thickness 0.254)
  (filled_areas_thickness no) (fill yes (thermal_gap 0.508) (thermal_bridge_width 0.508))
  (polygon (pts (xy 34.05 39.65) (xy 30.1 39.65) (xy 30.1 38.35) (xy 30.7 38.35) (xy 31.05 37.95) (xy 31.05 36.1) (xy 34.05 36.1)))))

